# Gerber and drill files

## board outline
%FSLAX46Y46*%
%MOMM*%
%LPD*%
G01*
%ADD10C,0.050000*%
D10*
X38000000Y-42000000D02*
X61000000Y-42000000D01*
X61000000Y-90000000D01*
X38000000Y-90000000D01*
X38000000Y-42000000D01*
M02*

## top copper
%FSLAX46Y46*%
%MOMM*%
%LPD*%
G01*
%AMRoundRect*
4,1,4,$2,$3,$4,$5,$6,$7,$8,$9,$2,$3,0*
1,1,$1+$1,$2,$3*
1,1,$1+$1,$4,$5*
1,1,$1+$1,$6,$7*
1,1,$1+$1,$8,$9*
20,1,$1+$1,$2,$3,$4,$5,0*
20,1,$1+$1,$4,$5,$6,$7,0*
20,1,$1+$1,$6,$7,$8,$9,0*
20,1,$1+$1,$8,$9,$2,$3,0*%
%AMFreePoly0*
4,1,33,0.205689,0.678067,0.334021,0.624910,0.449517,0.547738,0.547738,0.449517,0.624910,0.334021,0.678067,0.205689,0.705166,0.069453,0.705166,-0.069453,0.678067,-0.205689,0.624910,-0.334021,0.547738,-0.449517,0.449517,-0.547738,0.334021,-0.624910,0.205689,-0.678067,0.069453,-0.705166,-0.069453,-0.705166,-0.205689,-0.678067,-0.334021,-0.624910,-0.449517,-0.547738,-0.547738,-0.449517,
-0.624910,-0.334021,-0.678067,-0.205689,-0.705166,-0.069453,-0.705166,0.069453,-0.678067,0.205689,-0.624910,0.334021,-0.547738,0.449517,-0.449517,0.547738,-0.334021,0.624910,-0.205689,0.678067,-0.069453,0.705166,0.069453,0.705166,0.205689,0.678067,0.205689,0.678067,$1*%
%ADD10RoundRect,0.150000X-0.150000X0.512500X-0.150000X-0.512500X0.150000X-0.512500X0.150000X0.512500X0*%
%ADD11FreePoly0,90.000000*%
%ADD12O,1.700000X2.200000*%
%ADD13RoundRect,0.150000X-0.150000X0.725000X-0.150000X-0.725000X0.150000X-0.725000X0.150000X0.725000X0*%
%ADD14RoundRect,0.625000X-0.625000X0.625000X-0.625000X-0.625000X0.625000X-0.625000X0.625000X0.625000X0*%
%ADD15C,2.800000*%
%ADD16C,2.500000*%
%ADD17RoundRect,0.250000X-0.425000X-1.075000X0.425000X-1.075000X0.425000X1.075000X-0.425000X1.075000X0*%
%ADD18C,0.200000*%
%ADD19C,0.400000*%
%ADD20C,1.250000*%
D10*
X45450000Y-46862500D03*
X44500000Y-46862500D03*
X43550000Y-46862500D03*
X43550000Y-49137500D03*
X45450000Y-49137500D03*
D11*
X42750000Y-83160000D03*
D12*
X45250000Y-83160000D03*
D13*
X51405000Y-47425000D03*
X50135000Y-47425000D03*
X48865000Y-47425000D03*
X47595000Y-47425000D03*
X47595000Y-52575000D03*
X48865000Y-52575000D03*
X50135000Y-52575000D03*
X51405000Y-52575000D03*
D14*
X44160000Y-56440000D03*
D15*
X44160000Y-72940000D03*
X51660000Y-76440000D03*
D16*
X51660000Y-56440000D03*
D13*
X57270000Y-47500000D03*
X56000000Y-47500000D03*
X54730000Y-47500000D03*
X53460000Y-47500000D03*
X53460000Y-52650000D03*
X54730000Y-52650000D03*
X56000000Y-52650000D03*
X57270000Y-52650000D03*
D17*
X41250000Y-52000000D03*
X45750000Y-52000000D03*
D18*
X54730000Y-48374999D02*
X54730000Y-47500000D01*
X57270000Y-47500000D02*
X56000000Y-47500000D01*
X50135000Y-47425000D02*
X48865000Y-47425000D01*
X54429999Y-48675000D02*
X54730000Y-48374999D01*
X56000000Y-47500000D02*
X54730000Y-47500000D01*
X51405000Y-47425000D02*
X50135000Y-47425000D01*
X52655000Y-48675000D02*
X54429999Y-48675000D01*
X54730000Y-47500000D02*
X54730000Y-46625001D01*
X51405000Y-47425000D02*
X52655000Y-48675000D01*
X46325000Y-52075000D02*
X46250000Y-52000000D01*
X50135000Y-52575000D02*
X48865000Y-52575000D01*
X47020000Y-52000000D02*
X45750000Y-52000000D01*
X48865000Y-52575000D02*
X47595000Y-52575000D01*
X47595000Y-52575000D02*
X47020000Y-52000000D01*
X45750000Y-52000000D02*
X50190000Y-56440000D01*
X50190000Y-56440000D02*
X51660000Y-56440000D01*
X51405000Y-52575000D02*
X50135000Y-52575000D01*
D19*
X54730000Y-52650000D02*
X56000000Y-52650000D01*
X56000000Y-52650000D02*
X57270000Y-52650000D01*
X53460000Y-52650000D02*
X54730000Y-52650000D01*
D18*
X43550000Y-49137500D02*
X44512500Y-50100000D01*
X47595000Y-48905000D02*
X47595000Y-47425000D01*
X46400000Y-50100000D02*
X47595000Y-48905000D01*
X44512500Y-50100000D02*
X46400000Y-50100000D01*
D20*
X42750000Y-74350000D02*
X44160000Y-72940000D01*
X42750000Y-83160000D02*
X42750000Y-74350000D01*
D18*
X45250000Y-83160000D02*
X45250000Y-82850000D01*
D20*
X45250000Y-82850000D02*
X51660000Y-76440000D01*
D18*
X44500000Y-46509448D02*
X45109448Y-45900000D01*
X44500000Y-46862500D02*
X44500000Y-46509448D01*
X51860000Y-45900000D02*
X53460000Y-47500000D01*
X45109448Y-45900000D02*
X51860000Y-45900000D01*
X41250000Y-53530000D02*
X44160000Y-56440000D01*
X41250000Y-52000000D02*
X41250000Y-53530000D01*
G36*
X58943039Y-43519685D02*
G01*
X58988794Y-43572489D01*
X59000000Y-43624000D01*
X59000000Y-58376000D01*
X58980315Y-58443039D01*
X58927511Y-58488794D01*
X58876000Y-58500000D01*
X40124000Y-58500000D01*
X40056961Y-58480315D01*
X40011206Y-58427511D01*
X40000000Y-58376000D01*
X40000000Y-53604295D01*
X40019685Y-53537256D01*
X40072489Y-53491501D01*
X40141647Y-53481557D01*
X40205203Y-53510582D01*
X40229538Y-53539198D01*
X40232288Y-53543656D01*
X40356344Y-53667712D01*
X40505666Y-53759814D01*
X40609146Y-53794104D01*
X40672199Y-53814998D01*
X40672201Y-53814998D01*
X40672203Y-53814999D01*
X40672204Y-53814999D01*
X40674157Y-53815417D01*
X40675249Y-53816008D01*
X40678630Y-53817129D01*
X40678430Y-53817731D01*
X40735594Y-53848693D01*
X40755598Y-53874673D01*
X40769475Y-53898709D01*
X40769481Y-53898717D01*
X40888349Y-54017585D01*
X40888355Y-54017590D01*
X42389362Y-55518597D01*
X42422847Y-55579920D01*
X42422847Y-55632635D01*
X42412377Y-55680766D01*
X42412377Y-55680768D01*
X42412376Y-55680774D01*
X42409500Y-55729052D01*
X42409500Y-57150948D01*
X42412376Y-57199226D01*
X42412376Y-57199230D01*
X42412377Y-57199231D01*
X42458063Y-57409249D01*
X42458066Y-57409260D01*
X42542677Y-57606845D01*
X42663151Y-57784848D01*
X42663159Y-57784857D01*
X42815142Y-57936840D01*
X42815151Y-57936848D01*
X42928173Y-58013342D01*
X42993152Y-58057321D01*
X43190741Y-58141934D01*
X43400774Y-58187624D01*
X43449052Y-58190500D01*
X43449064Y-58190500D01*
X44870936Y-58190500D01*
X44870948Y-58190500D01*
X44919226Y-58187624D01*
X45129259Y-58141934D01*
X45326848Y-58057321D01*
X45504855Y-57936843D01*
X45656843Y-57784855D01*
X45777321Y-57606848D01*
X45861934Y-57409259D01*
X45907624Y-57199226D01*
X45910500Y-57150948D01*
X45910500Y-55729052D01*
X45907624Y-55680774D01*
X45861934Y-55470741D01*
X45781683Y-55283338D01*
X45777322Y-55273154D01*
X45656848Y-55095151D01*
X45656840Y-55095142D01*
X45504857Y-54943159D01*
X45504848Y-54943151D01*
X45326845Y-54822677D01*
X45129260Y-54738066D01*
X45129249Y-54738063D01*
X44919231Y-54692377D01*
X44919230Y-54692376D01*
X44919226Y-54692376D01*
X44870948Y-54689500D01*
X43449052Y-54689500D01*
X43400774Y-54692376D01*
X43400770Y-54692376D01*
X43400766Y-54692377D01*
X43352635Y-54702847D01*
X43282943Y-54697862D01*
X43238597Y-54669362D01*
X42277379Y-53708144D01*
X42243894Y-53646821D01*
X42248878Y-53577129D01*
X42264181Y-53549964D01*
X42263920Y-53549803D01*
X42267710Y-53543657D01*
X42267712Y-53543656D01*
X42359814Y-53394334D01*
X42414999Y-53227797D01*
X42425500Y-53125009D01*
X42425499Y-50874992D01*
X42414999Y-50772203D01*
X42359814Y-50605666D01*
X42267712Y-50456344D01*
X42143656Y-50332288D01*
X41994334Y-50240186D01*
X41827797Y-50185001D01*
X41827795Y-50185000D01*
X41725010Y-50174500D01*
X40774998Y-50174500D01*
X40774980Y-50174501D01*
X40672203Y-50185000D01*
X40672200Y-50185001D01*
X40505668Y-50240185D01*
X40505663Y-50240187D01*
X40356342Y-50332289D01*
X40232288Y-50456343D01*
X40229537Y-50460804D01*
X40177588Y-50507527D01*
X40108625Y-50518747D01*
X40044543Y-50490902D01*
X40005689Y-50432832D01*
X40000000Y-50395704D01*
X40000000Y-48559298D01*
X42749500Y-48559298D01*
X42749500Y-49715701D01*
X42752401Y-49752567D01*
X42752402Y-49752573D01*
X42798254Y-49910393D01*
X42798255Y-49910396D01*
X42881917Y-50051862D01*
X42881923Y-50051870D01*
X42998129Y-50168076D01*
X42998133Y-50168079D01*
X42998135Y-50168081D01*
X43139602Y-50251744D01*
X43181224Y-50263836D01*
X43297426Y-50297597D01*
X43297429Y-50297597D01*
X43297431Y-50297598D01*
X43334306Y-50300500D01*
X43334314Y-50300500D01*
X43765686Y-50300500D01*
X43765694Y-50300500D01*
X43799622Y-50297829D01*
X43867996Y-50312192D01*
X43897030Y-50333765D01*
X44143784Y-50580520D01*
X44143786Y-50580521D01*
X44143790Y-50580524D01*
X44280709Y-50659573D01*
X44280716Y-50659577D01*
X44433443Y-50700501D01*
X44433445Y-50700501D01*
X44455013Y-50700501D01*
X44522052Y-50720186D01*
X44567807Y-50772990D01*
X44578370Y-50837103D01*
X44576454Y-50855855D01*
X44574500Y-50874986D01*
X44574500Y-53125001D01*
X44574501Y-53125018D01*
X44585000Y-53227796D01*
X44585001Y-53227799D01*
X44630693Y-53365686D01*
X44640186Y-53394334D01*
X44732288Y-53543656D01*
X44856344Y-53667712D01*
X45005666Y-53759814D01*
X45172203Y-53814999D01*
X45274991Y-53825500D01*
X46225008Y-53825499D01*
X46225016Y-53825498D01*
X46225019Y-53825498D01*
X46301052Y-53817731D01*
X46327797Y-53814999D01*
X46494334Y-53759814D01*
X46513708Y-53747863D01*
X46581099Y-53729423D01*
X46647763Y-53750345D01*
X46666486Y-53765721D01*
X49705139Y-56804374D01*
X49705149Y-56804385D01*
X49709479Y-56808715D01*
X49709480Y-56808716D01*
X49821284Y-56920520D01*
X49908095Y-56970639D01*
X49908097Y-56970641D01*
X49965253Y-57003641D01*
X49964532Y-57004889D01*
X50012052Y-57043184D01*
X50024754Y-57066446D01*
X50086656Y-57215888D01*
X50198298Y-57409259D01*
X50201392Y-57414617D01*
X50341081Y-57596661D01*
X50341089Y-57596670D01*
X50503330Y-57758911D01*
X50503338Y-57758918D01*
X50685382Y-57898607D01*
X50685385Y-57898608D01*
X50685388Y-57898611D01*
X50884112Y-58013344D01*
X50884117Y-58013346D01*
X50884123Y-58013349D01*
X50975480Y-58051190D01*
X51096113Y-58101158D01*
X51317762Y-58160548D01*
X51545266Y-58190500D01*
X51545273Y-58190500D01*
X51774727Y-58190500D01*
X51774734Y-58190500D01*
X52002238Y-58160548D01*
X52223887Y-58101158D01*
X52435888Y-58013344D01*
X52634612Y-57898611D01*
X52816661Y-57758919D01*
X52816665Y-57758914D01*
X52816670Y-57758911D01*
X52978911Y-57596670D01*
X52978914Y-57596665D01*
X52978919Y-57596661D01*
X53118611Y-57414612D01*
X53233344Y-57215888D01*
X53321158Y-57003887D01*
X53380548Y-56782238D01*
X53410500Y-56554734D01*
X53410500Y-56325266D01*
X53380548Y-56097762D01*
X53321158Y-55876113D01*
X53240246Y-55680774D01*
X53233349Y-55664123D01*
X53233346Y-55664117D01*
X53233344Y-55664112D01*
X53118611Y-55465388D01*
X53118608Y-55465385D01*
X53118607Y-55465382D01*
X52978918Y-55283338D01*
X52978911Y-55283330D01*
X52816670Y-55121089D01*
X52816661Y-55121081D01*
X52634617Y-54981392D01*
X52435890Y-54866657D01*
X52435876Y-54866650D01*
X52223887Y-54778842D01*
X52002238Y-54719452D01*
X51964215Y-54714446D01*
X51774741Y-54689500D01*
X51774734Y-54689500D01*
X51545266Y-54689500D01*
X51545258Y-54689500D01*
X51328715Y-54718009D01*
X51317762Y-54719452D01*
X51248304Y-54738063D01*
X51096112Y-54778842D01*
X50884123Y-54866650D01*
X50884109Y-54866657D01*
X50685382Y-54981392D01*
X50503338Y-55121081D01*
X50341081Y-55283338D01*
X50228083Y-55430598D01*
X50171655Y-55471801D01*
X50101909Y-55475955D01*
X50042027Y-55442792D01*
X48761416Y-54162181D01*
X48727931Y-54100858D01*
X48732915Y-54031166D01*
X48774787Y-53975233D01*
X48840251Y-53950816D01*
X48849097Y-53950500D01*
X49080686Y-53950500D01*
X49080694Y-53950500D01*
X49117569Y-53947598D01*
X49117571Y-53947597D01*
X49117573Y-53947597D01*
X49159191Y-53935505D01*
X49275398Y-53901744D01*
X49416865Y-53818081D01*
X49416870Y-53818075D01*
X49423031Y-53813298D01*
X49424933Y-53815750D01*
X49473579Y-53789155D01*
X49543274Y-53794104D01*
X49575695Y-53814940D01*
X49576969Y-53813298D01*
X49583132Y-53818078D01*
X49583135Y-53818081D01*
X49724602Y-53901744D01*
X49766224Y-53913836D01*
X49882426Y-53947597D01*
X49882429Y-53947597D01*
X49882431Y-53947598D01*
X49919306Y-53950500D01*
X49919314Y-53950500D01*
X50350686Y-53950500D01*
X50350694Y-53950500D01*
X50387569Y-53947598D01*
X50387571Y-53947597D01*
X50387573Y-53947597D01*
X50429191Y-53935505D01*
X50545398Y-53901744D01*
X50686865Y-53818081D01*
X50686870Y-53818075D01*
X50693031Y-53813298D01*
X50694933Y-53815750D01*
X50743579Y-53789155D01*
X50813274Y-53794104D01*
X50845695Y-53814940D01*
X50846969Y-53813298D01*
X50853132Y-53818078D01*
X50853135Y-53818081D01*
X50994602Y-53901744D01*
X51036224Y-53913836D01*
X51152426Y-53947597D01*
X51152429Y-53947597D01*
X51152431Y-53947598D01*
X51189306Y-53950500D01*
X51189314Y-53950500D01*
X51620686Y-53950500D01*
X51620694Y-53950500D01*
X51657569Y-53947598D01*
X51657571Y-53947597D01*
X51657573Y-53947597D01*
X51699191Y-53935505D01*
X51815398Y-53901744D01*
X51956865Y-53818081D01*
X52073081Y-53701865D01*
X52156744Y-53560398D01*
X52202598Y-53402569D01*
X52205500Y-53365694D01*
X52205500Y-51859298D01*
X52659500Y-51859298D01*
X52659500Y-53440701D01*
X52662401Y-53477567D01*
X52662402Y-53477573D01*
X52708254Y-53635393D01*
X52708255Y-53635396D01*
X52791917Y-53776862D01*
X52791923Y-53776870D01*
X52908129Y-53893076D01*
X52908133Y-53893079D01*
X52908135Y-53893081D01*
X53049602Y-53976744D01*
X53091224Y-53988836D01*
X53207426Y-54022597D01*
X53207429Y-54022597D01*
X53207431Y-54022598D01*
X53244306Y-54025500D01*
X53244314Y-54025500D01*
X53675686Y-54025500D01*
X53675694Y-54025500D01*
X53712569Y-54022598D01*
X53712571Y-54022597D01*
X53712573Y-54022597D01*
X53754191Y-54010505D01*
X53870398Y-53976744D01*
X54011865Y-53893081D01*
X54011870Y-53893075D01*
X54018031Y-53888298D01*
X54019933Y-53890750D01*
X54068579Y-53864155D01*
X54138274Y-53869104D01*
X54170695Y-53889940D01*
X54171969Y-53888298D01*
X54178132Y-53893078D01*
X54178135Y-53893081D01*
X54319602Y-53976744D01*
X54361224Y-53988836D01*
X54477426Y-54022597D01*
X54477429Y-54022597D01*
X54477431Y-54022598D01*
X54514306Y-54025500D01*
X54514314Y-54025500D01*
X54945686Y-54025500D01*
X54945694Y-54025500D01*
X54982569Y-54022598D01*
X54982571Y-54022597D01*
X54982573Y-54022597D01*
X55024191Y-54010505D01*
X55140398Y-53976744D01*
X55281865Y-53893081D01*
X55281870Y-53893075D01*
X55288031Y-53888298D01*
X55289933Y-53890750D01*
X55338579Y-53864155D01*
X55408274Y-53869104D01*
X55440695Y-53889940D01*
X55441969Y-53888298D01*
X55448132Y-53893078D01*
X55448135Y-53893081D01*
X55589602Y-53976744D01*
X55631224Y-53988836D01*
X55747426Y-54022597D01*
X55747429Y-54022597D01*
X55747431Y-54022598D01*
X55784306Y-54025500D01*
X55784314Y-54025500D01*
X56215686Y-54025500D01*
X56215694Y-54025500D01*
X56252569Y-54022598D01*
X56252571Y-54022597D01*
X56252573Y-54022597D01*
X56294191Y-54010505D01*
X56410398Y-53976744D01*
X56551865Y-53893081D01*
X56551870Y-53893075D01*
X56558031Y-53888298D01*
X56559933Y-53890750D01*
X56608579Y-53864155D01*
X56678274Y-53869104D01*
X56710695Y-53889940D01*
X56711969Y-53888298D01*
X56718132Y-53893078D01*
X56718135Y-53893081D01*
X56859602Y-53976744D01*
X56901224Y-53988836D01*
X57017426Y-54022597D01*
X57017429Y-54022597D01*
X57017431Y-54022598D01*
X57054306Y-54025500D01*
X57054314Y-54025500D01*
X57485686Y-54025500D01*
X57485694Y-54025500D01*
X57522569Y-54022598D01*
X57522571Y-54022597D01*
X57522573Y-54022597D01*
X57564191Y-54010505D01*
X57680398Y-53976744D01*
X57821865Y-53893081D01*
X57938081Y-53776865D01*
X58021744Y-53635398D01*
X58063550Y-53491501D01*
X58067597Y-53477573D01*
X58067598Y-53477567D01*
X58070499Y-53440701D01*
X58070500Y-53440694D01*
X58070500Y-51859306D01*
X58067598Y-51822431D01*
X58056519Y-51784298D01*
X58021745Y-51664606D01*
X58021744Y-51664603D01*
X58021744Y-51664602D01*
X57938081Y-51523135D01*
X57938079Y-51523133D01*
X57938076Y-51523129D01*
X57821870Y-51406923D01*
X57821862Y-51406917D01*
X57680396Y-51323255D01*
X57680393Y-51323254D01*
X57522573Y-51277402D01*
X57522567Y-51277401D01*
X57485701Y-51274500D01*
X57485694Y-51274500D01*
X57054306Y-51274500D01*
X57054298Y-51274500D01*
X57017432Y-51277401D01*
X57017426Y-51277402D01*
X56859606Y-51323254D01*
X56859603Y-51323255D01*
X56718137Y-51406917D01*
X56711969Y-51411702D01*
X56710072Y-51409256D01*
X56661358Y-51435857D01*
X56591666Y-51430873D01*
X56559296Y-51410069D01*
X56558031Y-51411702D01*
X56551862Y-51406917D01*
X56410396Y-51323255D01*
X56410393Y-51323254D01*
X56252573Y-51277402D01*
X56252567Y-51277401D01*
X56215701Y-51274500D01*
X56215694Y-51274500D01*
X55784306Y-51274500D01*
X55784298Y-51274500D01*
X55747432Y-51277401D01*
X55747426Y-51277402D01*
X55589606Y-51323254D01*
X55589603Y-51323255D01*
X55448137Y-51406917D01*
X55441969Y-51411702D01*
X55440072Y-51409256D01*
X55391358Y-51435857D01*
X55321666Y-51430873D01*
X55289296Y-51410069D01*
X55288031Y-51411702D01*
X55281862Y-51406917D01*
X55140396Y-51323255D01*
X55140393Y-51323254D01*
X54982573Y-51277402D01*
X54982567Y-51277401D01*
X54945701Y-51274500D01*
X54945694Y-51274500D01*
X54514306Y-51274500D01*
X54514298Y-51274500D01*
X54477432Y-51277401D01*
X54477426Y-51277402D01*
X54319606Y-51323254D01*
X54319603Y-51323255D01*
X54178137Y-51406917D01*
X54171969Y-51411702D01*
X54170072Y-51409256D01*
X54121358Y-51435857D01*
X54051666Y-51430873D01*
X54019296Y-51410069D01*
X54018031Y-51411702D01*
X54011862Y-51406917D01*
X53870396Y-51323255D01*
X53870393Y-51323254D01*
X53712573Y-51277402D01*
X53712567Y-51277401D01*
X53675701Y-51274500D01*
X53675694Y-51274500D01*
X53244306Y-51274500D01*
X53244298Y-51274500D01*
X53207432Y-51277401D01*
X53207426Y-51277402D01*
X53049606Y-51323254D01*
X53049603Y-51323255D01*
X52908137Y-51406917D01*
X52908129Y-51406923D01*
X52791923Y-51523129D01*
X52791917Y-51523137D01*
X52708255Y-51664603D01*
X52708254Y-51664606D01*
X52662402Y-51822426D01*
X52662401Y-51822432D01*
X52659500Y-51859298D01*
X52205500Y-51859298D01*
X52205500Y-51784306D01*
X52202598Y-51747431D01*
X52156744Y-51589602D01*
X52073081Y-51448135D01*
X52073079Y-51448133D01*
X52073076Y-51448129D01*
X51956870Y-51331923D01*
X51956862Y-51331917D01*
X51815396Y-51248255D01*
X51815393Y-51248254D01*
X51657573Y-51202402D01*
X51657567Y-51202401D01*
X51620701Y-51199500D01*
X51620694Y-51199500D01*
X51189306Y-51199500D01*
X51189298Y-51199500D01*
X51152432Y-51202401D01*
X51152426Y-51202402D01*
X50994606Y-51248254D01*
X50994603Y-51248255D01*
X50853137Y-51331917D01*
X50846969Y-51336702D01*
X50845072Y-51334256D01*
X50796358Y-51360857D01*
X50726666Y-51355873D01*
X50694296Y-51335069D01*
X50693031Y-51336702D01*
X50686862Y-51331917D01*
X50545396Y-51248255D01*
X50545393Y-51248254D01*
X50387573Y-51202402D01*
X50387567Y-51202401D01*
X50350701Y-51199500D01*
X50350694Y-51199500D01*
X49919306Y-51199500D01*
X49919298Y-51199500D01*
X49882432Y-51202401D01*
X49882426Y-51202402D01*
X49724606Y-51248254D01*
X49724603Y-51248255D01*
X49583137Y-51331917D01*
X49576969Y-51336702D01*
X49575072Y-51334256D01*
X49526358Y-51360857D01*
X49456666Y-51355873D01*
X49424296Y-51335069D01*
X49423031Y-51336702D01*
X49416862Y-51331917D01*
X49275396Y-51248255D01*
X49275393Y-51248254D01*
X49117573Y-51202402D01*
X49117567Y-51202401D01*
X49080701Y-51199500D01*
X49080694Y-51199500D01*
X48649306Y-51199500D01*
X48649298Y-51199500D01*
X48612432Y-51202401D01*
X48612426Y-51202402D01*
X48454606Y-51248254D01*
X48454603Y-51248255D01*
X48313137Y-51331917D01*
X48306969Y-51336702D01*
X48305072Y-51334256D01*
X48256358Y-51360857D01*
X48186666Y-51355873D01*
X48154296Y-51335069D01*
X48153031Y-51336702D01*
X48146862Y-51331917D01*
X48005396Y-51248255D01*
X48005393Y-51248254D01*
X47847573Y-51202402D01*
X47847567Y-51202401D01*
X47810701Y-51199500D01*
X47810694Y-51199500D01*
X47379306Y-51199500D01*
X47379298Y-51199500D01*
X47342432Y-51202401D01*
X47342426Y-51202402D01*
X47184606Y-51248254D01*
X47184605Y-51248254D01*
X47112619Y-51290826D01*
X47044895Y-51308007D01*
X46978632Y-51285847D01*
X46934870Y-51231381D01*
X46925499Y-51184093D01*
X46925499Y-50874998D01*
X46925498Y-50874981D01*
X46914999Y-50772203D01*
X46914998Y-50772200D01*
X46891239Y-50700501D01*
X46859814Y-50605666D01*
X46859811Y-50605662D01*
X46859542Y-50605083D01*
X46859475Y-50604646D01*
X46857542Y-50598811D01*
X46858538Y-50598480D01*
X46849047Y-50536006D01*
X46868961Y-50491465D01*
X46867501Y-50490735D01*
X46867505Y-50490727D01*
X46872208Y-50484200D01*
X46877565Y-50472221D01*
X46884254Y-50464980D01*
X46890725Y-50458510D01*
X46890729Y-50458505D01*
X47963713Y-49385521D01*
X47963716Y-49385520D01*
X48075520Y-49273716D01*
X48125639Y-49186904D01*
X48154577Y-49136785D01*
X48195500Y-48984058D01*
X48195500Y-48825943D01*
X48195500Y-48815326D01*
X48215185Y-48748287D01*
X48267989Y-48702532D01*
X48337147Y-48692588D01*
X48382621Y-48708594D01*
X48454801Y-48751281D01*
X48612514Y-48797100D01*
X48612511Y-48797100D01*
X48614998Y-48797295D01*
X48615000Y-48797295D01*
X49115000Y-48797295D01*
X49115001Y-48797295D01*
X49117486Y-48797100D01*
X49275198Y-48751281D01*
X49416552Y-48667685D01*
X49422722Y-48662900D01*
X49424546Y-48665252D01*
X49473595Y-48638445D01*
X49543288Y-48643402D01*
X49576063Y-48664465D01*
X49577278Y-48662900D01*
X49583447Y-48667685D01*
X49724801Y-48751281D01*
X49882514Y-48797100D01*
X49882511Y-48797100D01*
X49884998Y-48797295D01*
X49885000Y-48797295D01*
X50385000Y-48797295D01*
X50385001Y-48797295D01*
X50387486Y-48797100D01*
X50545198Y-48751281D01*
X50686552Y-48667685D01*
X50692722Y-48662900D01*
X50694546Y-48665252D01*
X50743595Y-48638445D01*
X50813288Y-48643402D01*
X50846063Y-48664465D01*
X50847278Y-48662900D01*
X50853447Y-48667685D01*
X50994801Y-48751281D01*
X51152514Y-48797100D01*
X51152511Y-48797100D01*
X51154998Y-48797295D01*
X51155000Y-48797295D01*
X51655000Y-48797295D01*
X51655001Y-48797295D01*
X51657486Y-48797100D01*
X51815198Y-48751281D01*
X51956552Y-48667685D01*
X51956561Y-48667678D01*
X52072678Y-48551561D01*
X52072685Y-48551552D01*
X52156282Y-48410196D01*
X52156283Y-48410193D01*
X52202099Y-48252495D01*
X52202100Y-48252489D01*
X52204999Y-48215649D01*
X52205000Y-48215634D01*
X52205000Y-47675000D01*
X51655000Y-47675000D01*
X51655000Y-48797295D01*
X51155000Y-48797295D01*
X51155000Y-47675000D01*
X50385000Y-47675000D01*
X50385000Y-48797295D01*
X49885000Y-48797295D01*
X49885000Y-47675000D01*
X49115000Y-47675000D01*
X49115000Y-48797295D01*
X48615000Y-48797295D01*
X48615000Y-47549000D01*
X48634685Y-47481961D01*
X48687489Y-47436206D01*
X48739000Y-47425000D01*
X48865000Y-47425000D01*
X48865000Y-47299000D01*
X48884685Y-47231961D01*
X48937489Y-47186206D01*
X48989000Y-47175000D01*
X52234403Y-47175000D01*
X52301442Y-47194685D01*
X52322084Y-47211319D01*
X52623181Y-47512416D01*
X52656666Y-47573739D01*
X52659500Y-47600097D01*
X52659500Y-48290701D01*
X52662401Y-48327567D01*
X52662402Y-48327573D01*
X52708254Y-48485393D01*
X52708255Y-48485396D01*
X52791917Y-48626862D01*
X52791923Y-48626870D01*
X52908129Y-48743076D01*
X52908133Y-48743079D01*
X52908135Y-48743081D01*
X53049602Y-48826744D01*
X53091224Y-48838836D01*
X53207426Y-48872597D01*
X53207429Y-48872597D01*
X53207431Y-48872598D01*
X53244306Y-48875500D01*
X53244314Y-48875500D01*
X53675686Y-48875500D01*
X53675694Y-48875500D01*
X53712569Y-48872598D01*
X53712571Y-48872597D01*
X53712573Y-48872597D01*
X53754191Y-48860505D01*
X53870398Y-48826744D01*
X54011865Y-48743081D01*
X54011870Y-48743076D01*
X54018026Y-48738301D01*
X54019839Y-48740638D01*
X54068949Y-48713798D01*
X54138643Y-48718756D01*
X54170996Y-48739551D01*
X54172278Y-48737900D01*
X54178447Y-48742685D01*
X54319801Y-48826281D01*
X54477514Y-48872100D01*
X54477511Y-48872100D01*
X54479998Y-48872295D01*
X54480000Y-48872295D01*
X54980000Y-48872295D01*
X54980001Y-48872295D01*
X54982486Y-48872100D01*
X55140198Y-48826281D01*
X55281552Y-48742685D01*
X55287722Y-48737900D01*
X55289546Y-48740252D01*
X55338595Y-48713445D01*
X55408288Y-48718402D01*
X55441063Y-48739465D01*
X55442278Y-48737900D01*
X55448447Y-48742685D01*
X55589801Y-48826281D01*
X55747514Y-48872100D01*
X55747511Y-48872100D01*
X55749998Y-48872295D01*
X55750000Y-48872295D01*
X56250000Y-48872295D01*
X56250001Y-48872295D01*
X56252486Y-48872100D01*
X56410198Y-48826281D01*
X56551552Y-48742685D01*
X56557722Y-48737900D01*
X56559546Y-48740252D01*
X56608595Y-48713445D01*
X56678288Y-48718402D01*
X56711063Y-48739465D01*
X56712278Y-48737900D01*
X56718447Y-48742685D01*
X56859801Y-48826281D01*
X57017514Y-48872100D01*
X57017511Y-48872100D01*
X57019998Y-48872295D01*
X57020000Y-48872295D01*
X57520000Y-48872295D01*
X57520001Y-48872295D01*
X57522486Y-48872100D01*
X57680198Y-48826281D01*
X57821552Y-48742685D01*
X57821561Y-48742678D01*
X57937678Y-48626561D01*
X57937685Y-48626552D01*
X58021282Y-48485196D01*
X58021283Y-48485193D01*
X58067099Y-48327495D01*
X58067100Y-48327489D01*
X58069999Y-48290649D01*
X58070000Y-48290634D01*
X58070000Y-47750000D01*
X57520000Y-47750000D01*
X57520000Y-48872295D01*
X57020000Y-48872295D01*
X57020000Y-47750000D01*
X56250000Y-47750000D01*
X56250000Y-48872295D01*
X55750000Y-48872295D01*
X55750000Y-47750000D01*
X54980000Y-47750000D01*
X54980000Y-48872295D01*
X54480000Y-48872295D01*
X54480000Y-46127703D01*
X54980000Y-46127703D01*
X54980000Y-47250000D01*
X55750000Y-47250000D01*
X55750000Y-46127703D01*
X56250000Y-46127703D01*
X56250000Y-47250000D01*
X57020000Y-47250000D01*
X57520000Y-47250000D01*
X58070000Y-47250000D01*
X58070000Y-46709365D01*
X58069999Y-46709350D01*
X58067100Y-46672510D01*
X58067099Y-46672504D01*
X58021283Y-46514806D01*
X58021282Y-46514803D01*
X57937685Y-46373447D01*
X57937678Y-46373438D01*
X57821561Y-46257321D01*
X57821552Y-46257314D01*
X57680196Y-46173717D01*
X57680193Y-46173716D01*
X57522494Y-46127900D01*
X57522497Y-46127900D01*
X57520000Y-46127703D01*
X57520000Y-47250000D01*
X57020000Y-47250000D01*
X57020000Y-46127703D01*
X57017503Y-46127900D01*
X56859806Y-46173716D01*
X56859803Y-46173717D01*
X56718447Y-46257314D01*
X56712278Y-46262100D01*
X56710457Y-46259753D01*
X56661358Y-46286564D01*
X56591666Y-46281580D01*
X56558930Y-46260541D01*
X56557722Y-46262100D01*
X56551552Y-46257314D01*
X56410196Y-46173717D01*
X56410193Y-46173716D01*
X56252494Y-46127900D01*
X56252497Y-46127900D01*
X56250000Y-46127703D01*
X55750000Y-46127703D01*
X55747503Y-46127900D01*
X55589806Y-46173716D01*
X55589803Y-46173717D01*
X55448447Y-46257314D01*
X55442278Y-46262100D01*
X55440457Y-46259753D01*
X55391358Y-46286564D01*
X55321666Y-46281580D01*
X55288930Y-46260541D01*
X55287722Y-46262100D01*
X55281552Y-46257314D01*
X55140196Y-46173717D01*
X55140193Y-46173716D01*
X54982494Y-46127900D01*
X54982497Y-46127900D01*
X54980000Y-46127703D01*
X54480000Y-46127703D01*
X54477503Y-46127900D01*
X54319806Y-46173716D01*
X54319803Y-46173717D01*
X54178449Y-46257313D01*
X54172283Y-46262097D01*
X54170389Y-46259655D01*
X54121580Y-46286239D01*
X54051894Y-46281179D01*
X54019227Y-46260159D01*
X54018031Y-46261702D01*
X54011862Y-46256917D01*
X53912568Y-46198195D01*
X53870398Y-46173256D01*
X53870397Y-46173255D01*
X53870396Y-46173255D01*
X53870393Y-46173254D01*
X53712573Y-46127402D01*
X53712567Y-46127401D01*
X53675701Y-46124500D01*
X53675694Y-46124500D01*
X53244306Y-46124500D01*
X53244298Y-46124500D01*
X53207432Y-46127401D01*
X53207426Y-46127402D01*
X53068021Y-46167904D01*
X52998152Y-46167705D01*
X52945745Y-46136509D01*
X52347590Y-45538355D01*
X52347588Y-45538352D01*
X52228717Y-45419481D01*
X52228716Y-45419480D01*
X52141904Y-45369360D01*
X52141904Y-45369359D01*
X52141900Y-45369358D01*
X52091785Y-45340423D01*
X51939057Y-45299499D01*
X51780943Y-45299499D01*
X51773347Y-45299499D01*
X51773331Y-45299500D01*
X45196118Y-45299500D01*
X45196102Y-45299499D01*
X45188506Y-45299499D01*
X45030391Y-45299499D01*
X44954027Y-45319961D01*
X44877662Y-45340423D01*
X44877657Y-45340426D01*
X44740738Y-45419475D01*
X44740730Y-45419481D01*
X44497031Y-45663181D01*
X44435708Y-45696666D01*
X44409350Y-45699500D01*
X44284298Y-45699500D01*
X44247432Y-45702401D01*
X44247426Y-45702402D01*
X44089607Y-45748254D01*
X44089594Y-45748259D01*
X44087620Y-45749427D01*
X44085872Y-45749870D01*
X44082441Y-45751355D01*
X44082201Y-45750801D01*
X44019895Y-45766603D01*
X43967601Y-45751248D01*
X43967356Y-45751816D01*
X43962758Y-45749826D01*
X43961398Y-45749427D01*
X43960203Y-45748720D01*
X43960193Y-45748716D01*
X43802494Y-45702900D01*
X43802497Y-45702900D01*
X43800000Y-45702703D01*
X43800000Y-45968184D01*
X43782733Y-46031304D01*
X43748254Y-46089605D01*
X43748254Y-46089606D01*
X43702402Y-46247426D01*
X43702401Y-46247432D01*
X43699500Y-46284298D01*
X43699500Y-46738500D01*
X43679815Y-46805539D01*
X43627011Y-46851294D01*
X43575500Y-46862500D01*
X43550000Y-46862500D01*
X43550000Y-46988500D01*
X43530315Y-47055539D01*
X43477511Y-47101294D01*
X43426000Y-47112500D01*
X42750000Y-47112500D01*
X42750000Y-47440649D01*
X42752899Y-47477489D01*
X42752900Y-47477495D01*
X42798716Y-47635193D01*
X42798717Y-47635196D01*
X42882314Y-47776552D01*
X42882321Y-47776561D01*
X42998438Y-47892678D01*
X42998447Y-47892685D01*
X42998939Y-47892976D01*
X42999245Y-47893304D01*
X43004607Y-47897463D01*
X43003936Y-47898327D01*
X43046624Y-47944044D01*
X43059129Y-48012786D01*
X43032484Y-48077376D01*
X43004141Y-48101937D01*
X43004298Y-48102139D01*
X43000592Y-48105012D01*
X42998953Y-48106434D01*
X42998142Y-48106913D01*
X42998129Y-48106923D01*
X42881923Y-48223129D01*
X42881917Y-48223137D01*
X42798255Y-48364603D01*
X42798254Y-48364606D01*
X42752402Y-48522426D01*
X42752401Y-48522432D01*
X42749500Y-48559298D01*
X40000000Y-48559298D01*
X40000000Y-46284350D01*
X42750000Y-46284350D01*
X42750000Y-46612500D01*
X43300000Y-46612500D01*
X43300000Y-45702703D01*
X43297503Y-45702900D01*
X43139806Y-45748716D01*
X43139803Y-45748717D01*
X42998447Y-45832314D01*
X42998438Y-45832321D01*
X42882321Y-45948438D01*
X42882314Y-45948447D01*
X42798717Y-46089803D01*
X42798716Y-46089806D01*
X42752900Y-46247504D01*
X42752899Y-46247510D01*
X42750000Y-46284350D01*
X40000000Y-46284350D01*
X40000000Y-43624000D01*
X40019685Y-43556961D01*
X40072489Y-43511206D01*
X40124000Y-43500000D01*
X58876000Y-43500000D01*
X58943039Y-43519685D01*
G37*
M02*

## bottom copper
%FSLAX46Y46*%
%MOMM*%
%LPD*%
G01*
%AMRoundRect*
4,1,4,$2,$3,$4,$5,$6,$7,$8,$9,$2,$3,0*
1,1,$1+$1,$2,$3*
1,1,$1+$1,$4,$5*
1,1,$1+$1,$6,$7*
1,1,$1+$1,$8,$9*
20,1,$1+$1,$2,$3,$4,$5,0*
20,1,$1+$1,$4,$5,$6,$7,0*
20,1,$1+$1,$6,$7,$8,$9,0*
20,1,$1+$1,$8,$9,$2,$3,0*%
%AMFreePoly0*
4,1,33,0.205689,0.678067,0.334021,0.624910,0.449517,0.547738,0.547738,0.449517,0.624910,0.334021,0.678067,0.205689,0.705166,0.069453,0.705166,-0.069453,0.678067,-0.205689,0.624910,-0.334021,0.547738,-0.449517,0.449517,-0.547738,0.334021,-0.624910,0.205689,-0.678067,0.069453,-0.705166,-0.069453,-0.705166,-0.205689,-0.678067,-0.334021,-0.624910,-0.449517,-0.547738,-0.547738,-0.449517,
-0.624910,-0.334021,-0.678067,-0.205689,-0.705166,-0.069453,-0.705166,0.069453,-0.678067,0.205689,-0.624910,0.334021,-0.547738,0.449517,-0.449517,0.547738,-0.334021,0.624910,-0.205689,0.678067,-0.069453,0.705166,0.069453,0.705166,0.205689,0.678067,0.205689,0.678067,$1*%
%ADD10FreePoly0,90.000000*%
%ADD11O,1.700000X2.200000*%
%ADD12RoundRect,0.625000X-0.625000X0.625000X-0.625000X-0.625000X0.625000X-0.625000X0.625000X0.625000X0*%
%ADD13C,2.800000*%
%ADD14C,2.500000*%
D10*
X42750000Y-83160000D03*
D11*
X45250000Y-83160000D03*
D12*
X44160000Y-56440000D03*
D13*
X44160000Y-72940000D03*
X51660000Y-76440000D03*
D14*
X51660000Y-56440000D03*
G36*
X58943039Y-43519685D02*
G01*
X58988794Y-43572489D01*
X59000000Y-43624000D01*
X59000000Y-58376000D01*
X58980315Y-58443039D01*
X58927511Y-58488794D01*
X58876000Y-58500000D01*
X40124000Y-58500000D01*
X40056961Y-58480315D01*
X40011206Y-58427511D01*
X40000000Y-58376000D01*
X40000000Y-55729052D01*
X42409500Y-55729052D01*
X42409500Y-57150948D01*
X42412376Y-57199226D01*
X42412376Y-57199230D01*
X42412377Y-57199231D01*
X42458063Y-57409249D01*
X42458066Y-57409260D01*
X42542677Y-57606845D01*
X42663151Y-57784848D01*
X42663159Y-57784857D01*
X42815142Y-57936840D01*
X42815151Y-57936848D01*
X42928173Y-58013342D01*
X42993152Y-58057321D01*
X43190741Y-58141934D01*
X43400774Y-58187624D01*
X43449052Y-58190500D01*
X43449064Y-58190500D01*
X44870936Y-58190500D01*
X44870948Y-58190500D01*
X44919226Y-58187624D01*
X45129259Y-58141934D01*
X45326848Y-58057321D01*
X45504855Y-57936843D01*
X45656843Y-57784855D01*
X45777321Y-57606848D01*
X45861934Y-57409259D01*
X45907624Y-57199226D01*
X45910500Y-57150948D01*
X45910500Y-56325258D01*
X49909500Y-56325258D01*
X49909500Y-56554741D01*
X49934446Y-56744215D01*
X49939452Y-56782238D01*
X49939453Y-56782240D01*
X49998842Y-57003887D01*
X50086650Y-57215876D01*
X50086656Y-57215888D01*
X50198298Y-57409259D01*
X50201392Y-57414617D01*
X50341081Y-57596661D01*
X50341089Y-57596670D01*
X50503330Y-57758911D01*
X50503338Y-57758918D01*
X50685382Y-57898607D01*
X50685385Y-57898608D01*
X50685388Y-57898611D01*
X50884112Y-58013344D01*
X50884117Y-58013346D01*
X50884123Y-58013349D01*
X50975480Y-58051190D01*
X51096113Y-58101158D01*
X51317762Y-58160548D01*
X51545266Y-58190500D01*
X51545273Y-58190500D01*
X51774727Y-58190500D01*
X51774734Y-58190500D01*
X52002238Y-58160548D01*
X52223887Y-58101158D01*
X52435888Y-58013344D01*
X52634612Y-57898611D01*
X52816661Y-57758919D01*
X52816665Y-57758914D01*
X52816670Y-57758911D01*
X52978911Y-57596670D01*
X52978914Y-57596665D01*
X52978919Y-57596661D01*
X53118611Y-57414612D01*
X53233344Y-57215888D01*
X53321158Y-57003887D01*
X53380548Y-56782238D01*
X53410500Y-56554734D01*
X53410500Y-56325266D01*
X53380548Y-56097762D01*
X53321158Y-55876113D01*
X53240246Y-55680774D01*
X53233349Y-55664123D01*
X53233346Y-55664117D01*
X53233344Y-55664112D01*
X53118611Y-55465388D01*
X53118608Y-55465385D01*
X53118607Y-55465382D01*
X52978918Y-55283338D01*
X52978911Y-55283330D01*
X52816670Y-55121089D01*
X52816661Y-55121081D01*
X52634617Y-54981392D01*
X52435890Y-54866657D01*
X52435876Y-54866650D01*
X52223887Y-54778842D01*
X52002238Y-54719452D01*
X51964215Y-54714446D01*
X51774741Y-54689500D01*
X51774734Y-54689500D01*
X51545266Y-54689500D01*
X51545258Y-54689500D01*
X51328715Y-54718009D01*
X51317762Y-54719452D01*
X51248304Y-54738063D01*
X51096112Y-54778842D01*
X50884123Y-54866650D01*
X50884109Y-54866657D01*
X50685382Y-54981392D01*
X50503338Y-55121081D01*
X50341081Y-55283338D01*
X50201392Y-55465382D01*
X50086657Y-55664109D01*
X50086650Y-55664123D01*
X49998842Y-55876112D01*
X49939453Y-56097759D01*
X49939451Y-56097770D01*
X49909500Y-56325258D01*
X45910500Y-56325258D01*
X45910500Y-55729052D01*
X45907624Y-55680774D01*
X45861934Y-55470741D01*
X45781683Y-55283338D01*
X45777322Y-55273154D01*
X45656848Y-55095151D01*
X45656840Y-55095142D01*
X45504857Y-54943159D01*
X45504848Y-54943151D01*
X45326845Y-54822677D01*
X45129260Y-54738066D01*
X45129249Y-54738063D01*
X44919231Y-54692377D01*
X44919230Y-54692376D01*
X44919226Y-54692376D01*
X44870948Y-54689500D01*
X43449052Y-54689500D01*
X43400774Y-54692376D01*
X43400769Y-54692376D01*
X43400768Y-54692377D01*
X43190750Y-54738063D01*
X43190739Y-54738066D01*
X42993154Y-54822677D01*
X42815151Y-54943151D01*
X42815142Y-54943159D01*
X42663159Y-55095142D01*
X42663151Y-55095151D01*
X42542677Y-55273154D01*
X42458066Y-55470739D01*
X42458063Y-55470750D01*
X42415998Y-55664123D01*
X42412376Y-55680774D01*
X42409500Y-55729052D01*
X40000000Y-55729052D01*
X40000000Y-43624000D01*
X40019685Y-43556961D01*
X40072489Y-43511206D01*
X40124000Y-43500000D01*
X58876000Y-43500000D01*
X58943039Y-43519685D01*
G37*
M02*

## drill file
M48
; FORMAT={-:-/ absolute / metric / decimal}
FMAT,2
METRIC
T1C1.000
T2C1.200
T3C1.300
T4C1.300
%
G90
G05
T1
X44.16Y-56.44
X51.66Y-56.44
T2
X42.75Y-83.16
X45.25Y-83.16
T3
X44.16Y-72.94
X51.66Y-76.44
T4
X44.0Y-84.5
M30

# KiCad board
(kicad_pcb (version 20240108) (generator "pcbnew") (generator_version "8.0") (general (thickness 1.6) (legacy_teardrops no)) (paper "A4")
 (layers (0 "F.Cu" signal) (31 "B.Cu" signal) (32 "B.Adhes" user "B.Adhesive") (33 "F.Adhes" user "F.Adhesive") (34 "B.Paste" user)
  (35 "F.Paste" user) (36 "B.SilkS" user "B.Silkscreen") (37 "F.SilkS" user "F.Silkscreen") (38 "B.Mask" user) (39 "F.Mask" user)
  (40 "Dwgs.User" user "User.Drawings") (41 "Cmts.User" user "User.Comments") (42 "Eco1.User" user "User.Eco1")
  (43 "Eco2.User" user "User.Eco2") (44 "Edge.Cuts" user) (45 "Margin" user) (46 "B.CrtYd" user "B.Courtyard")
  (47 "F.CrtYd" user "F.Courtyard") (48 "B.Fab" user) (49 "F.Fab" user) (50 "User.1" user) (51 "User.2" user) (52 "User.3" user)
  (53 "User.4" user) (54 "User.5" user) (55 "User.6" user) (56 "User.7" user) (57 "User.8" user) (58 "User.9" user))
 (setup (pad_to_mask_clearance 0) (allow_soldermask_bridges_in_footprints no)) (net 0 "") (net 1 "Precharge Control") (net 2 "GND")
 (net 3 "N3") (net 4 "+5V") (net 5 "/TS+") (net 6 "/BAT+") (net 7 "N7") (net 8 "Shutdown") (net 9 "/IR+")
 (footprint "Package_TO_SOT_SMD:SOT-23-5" (layer "F.Cu") (at 44.5 48 -90)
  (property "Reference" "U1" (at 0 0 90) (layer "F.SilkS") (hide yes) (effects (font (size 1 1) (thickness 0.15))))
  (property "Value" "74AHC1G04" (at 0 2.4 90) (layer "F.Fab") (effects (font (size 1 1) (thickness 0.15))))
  (pad "1" smd roundrect (at -1.1375 -0.95 270) (size 1.325 0.6) (layers "F.Cu" "F.Paste" "F.Mask") (roundrect_rratio 0.25))
  (pad "2" smd roundrect (at -1.1375 0 270) (size 1.325 0.6) (layers "F.Cu" "F.Paste" "F.Mask") (roundrect_rratio 0.25)
   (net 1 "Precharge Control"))
  (pad "3" smd roundrect (at -1.1375 0.95 270) (size 1.325 0.6) (layers "F.Cu" "F.Paste" "F.Mask") (roundrect_rratio 0.25) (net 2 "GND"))
  (pad "4" smd roundrect (at 1.1375 0.95 270) (size 1.325 0.6) (layers "F.Cu" "F.Paste" "F.Mask") (roundrect_rratio 0.25) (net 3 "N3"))
  (pad "5" smd roundrect (at 1.1375 -0.95 270) (size 1.325 0.6) (layers "F.Cu" "F.Paste" "F.Mask") (roundrect_rratio 0.25) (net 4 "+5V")))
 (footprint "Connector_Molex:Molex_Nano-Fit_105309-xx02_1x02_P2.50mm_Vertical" (layer "F.Cu") (at 42.75 83.16 90)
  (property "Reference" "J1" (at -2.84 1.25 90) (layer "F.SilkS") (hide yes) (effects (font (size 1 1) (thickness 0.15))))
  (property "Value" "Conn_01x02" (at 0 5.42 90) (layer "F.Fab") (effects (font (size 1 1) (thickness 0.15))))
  (pad "" np_thru_hole circle (at -1.34 1.25 90) (size 1.3 1.3) (drill 1.3) (layers "*.Cu" "*.Mask"))
  (pad "1" thru_hole custom (at 0 0 90) (size 1.417157 1.417157) (drill 1.2) (layers "*.Cu" "*.Mask") (remove_unused_layers no)
   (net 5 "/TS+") (thermal_bridge_angle 90) (options (clearance outline) (anchor circle)) (primitives))
  (pad "2" thru_hole oval (at 0 2.5 90) (size 2.2 1.7) (drill 1.2) (layers "*.Cu" "*.Mask") (remove_unused_layers no) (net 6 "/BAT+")))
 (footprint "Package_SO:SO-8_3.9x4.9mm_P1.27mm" (layer "F.Cu") (at 49.5 50 -90)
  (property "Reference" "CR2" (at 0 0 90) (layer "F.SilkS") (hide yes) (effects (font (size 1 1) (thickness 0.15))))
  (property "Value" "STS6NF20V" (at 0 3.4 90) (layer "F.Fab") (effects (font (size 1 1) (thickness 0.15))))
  (pad "1" smd roundrect (at -2.575 -1.905 270) (size 1.75 0.6) (layers "F.Cu" "F.Paste" "F.Mask") (roundrect_rratio 0.25) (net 2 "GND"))
  (pad "2" smd roundrect (at -2.575 -0.635 270) (size 1.75 0.6) (layers "F.Cu" "F.Paste" "F.Mask") (roundrect_rratio 0.25) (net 2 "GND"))
  (pad "3" smd roundrect (at -2.575 0.635 270) (size 1.75 0.6) (layers "F.Cu" "F.Paste" "F.Mask") (roundrect_rratio 0.25) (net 2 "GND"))
  (pad "4" smd roundrect (at -2.575 1.905 270) (size 1.75 0.6) (layers "F.Cu" "F.Paste" "F.Mask") (roundrect_rratio 0.25) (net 3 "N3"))
  (pad "5" smd roundrect (at 2.575 1.905 270) (size 1.75 0.6) (layers "F.Cu" "F.Paste" "F.Mask") (roundrect_rratio 0.25) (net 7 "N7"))
  (pad "6" smd roundrect (at 2.575 0.635 270) (size 1.75 0.6) (layers "F.Cu" "F.Paste" "F.Mask") (roundrect_rratio 0.25) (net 7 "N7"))
  (pad "7" smd roundrect (at 2.575 -0.635 270) (size 1.75 0.6) (layers "F.Cu" "F.Paste" "F.Mask") (roundrect_rratio 0.25) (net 7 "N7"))
  (pad "8" smd roundrect (at 2.575 -1.905 270) (size 1.75 0.6) (layers "F.Cu" "F.Paste" "F.Mask") (roundrect_rratio 0.25) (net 7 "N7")))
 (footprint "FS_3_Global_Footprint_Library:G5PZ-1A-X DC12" (layer "F.Cu") (at 55.5 53.9 -90)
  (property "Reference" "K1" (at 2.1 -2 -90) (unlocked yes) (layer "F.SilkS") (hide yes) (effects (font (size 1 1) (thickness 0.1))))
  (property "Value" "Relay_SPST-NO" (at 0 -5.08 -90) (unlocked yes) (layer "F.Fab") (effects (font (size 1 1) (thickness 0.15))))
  (pad "1" thru_hole roundrect (at 2.54 11.34 270) (size 2.5 2.5) (drill 1) (layers "*.Cu" "*.Mask") (remove_unused_layers no)
   (roundrect_rratio 0.25) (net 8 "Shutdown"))
  (pad "2" thru_hole circle (at 19.04 11.34 270) (size 2.8 2.8) (drill 1.3) (layers "*.Cu" "*.Mask") (remove_unused_layers no)
   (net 5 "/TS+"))
  (pad "3" thru_hole circle (at 22.54 3.84 270) (size 2.8 2.8) (drill 1.3) (layers "*.Cu" "*.Mask") (remove_unused_layers no)
   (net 6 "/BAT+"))
  (pad "4" thru_hole circle (at 2.54 3.84 270) (size 2.5 2.5) (drill 1) (layers "*.Cu" "*.Mask") (remove_unused_layers no) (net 7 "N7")))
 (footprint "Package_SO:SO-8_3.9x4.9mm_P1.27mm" (layer "F.Cu") (at 55.365 50.075 -90)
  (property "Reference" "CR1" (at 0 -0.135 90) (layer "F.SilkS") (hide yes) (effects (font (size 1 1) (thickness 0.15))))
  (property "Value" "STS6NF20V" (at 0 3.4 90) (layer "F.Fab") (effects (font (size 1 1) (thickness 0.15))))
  (pad "1" smd roundrect (at -2.575 -1.905 270) (size 1.75 0.6) (layers "F.Cu" "F.Paste" "F.Mask") (roundrect_rratio 0.25) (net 2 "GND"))
  (pad "2" smd roundrect (at -2.575 -0.635 270) (size 1.75 0.6) (layers "F.Cu" "F.Paste" "F.Mask") (roundrect_rratio 0.25) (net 2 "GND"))
  (pad "3" smd roundrect (at -2.575 0.635 270) (size 1.75 0.6) (layers "F.Cu" "F.Paste" "F.Mask") (roundrect_rratio 0.25) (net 2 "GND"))
  (pad "4" smd roundrect (at -2.575 1.905 270) (size 1.75 0.6) (layers "F.Cu" "F.Paste" "F.Mask") (roundrect_rratio 0.25)
   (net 1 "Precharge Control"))
  (pad "5" smd roundrect (at 2.575 1.905 270) (size 1.75 0.6) (layers "F.Cu" "F.Paste" "F.Mask") (roundrect_rratio 0.25) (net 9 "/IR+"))
  (pad "6" smd roundrect (at 2.575 0.635 270) (size 1.75 0.6) (layers "F.Cu" "F.Paste" "F.Mask") (roundrect_rratio 0.25) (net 9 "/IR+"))
  (pad "7" smd roundrect (at 2.575 -0.635 270) (size 1.75 0.6) (layers "F.Cu" "F.Paste" "F.Mask") (roundrect_rratio 0.25) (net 9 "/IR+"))
  (pad "8" smd roundrect (at 2.575 -1.905 270) (size 1.75 0.6) (layers "F.Cu" "F.Paste" "F.Mask") (roundrect_rratio 0.25) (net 9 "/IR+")))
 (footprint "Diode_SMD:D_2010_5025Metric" (layer "F.Cu") (at 43.5 52)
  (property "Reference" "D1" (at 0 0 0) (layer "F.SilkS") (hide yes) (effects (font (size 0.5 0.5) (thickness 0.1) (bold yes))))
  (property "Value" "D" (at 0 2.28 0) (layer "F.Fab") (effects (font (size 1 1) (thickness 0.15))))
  (pad "1" smd roundrect (at -2.25 0) (size 1.35 2.65) (layers "F.Cu" "F.Paste" "F.Mask") (roundrect_rratio 0.185185) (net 8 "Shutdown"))
  (pad "2" smd roundrect (at 2.25 0) (size 1.35 2.65) (layers "F.Cu" "F.Paste" "F.Mask") (roundrect_rratio 0.185185) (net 7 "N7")))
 (gr_rect (start 38 42) (end 61 90) (stroke (width 0.05) (type default)) (fill none) (layer "Edge.Cuts"))
 (segment (start 54.73 48.374999) (end 54.73 47.5) (width 0.2) (layer "F.Cu") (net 2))
 (segment (start 57.27 47.5) (end 56 47.5) (width 0.2) (layer "F.Cu") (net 2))
 (segment (start 50.135 47.425) (end 48.865 47.425) (width 0.2) (layer "F.Cu") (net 2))
 (segment (start 54.429999 48.675) (end 54.73 48.374999) (width 0.2) (layer "F.Cu") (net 2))
 (segment (start 56 47.5) (end 54.73 47.5) (width 0.2) (layer "F.Cu") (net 2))
 (segment (start 51.405 47.425) (end 50.135 47.425) (width 0.2) (layer "F.Cu") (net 2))
 (segment (start 52.655 48.675) (end 54.429999 48.675) (width 0.2) (layer "F.Cu") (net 2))
 (segment (start 54.73 47.5) (end 54.73 46.625001) (width 0.2) (layer "F.Cu") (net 2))
 (segment (start 51.405 47.425) (end 52.655 48.675) (width 0.2) (layer "F.Cu") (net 2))
 (segment (start 46.325 52.075) (end 46.25 52) (width 0.2) (layer "F.Cu") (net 7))
 (segment (start 50.135 52.575) (end 48.865 52.575) (width 0.2) (layer "F.Cu") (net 7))
 (segment (start 47.02 52) (end 45.75 52) (width 0.2) (layer "F.Cu") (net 7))
 (segment (start 48.865 52.575) (end 47.595 52.575) (width 0.2) (layer "F.Cu") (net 7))
 (segment (start 47.595 52.575) (end 47.02 52) (width 0.2) (layer "F.Cu") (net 7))
 (segment (start 45.75 52) (end 50.19 56.44) (width 0.2) (layer "F.Cu") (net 7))
 (segment (start 50.19 56.44) (end 51.66 56.44) (width 0.2) (layer "F.Cu") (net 7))
 (segment (start 51.405 52.575) (end 50.135 52.575) (width 0.2) (layer "F.Cu") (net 7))
 (segment (start 54.73 52.65) (end 56 52.65) (width 0.4) (layer "F.Cu") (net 9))
 (segment (start 56 52.65) (end 57.27 52.65) (width 0.4) (layer "F.Cu") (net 9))
 (segment (start 53.46 52.65) (end 54.73 52.65) (width 0.4) (layer "F.Cu") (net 9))
 (segment (start 43.55 49.1375) (end 44.5125 50.1) (width 0.2) (layer "F.Cu") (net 3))
 (segment (start 47.595 48.905) (end 47.595 47.425) (width 0.2) (layer "F.Cu") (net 3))
 (segment (start 46.4 50.1) (end 47.595 48.905) (width 0.2) (layer "F.Cu") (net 3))
 (segment (start 44.5125 50.1) (end 46.4 50.1) (width 0.2) (layer "F.Cu") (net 3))
 (segment (start 42.75 74.35) (end 44.16 72.94) (width 1.25) (layer "F.Cu") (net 5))
 (segment (start 42.75 83.16) (end 42.75 74.35) (width 1.25) (layer "F.Cu") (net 5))
 (segment (start 45.25 83.16) (end 45.25 82.85) (width 0.2) (layer "F.Cu") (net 6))
 (segment (start 45.25 82.85) (end 51.66 76.44) (width 1.25) (layer "F.Cu") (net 6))
 (segment (start 44.5 46.509448) (end 45.109448 45.9) (width 0.2) (layer "F.Cu") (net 1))
 (segment (start 44.5 46.8625) (end 44.5 46.509448) (width 0.2) (layer "F.Cu") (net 1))
 (segment (start 51.86 45.9) (end 53.46 47.5) (width 0.2) (layer "F.Cu") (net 1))
 (segment (start 45.109448 45.9) (end 51.86 45.9) (width 0.2) (layer "F.Cu") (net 1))
 (segment (start 41.25 53.53) (end 44.16 56.44) (width 0.2) (layer "F.Cu") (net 8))
 (segment (start 41.25 52) (end 41.25 53.53) (width 0.2) (layer "F.Cu") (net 8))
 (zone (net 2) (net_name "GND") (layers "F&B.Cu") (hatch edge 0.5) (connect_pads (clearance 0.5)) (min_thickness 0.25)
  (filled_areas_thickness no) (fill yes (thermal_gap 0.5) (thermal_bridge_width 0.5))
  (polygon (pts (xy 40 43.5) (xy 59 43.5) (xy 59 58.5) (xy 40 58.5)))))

